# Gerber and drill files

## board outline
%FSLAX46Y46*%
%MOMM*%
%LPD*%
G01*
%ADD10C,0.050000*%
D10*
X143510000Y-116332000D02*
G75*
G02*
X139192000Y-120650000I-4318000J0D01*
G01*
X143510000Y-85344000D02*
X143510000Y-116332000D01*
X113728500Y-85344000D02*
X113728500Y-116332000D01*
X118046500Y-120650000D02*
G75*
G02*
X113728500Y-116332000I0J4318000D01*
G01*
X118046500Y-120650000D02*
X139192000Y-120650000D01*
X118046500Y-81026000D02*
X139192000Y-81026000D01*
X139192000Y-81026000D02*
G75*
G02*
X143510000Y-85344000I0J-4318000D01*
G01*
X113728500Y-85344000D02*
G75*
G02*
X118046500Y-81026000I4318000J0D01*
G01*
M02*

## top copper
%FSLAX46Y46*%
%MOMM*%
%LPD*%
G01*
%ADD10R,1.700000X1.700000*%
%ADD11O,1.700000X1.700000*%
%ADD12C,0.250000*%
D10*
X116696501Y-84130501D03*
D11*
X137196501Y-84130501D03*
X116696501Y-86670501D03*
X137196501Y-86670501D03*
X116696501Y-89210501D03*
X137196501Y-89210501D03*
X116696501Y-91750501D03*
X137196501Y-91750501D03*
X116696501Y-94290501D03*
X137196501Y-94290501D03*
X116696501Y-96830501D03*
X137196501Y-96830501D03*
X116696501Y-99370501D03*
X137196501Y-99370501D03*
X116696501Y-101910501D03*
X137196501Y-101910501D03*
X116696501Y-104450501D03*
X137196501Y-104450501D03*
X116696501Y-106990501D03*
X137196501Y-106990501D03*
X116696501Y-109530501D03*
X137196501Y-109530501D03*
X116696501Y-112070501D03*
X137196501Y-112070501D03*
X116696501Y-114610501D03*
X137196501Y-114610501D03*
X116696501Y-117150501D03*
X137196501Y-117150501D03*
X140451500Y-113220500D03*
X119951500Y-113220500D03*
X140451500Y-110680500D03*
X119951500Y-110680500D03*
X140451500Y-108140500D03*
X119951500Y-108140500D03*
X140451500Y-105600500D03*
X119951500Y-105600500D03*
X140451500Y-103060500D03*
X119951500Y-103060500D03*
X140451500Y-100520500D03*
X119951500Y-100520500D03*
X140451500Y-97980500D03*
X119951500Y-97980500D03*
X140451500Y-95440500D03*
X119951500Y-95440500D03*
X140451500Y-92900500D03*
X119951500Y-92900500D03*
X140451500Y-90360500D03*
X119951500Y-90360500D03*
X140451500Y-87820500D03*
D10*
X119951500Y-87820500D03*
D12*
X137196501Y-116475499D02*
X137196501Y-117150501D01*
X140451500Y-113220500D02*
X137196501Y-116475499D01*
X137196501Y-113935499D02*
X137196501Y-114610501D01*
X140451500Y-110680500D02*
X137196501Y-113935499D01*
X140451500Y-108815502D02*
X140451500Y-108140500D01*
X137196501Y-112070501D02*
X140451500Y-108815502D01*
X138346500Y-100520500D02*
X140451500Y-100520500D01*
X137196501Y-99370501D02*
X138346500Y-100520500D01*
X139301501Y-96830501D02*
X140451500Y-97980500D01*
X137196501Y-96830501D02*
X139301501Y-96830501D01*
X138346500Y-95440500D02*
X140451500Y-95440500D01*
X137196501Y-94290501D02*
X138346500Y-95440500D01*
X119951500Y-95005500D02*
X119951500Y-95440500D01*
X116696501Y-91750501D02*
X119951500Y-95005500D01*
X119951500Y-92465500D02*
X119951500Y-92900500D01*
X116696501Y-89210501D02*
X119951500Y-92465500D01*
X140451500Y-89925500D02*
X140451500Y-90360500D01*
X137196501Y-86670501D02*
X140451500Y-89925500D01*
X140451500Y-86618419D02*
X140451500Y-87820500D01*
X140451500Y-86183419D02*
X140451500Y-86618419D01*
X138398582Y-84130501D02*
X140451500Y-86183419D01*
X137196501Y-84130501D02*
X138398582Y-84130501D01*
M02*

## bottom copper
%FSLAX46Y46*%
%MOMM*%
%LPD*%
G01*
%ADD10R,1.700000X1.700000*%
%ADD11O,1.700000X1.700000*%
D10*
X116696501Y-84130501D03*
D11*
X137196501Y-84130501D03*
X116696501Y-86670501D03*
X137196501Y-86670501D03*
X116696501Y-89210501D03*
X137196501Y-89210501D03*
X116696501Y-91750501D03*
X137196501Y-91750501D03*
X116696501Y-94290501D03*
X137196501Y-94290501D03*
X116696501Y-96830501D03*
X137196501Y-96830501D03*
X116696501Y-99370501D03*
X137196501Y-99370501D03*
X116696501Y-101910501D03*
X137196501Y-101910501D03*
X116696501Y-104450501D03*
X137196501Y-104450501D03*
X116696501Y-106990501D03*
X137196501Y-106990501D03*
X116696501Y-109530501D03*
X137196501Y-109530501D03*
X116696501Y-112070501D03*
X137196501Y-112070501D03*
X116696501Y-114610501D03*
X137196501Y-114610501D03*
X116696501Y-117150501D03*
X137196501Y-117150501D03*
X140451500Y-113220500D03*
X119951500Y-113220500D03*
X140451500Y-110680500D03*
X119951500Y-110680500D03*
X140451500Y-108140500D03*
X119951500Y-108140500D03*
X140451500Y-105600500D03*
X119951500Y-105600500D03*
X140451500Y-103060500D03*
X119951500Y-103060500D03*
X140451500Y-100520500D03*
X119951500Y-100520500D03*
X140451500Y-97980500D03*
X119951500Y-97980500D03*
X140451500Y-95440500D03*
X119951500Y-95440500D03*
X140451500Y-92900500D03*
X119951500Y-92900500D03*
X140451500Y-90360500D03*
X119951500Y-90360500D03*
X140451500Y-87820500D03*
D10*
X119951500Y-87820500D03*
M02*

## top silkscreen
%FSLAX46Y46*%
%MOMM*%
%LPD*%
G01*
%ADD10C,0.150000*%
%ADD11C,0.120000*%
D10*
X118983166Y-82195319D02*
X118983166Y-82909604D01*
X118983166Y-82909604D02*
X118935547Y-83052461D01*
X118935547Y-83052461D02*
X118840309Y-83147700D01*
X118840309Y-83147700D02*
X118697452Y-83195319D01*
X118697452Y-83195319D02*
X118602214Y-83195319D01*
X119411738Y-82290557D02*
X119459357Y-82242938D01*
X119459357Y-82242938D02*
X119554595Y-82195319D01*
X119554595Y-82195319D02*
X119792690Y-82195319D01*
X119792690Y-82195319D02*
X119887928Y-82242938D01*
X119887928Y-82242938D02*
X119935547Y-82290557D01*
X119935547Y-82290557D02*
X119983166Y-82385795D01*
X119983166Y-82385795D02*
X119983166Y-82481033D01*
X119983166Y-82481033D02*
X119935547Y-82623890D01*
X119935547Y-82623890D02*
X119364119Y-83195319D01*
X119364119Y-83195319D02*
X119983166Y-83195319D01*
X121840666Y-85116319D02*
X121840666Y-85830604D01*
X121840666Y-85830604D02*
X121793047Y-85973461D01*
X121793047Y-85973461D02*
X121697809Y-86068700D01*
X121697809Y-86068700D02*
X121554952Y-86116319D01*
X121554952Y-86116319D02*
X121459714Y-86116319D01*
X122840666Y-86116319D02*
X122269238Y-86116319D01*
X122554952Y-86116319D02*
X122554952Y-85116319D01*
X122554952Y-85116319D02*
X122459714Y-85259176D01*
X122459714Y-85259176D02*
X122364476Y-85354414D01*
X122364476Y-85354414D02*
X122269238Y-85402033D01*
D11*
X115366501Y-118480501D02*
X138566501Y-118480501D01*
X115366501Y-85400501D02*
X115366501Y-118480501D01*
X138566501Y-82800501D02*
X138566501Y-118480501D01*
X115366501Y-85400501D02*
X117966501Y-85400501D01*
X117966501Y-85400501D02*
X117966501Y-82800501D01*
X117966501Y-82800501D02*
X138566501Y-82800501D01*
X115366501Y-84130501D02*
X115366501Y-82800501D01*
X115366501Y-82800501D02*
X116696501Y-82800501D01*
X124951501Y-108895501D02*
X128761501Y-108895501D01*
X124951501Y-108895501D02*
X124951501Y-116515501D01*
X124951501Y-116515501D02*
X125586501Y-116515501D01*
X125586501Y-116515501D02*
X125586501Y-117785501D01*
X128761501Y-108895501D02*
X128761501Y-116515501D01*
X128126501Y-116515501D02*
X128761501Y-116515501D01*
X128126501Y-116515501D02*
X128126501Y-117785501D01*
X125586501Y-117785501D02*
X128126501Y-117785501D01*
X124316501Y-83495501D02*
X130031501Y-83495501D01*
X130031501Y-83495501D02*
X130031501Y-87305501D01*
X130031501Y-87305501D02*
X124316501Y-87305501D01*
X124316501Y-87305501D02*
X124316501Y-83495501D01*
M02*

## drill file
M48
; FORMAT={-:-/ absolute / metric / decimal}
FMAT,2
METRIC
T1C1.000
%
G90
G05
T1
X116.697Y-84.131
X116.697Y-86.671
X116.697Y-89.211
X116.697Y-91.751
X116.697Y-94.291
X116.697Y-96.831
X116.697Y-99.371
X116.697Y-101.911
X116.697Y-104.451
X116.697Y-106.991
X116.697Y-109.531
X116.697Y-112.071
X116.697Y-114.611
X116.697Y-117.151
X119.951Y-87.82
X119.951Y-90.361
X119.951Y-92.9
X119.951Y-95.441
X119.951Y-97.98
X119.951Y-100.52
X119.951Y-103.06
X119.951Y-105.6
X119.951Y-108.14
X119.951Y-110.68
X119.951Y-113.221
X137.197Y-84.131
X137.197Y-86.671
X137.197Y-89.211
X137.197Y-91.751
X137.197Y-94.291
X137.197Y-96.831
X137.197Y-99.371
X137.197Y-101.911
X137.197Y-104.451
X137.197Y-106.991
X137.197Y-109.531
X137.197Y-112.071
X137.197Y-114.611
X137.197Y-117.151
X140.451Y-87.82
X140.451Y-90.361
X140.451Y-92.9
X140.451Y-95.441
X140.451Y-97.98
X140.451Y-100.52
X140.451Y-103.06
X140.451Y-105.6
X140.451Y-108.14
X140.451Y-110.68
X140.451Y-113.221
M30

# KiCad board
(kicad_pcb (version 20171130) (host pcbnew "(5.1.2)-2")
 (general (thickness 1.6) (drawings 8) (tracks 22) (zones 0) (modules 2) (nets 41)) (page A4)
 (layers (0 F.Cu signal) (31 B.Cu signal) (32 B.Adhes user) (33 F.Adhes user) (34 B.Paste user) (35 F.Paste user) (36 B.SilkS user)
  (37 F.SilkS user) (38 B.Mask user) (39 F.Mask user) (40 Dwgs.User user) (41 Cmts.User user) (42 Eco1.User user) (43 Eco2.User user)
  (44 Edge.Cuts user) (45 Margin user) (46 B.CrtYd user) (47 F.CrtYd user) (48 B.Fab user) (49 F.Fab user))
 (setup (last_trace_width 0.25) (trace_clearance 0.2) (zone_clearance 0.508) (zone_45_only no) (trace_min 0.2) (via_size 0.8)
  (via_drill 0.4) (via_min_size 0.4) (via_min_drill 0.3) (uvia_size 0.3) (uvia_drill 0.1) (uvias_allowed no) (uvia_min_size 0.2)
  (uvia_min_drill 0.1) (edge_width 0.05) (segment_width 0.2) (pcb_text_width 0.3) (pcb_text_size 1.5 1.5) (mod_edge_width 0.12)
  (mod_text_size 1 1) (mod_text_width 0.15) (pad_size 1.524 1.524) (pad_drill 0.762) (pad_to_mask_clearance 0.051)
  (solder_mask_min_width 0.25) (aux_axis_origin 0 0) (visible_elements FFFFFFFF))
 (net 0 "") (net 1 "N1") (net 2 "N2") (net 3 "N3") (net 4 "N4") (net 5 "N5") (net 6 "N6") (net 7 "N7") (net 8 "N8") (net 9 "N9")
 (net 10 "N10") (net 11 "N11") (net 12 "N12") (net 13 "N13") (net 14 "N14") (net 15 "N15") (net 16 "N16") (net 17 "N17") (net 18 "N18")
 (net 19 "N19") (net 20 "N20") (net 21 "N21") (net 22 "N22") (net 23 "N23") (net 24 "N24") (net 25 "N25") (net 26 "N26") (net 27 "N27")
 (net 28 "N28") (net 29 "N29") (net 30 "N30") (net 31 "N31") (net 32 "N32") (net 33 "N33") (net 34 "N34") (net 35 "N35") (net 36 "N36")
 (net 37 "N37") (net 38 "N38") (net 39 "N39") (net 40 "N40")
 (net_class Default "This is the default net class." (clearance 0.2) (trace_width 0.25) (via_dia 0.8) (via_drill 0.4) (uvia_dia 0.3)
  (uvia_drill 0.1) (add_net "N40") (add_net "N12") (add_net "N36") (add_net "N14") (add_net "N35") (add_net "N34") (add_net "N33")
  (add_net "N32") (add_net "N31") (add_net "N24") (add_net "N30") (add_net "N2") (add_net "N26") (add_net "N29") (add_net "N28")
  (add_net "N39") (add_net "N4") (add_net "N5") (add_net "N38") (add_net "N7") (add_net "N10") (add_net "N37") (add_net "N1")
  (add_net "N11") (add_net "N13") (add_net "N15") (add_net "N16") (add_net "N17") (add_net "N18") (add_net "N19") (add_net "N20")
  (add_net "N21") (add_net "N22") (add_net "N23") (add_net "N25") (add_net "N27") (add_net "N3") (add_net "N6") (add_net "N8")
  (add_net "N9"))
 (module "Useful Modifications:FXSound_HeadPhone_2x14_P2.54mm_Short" (layer F.Cu) (at 116.696501 84.130501)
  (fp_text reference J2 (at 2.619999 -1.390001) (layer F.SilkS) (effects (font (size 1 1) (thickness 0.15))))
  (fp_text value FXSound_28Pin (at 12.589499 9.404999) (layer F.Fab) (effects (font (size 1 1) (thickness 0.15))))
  (fp_line (start -1.33 34.35) (end 21.87 34.35) (layer F.SilkS) (width 0.12))
  (fp_line (start -1.33 1.27) (end -1.33 34.35) (layer F.SilkS) (width 0.12))
  (fp_line (start 21.87 -1.33) (end 21.87 34.35) (layer F.SilkS) (width 0.12))
  (fp_line (start -1.33 1.27) (end 1.27 1.27) (layer F.SilkS) (width 0.12))
  (fp_line (start 1.27 1.27) (end 1.27 -1.33) (layer F.SilkS) (width 0.12))
  (fp_line (start 1.27 -1.33) (end 21.87 -1.33) (layer F.SilkS) (width 0.12))
  (fp_line (start -1.33 0) (end -1.33 -1.33) (layer F.SilkS) (width 0.12))
  (fp_line (start -1.33 -1.33) (end 0 -1.33) (layer F.SilkS) (width 0.12))
  (fp_line (start 8.255 24.765) (end 12.065 24.765) (layer F.SilkS) (width 0.12))
  (fp_line (start 8.255 24.765) (end 8.255 32.385) (layer F.SilkS) (width 0.12))
  (fp_line (start 8.255 32.385) (end 8.89 32.385) (layer F.SilkS) (width 0.12))
  (fp_line (start 8.89 32.385) (end 8.89 33.655) (layer F.SilkS) (width 0.12))
  (fp_line (start 12.065 24.765) (end 12.065 32.385) (layer F.SilkS) (width 0.12))
  (fp_line (start 11.43 32.385) (end 12.065 32.385) (layer F.SilkS) (width 0.12))
  (fp_line (start 11.43 32.385) (end 11.43 33.655) (layer F.SilkS) (width 0.12))
  (fp_line (start 8.89 33.655) (end 11.43 33.655) (layer F.SilkS) (width 0.12))
  (fp_line (start 7.62 -0.635) (end 13.335 -0.635) (layer F.SilkS) (width 0.12))
  (fp_line (start 13.335 -0.635) (end 13.335 3.175) (layer F.SilkS) (width 0.12))
  (fp_line (start 13.335 3.175) (end 7.62 3.175) (layer F.SilkS) (width 0.12))
  (fp_line (start 7.62 3.175) (end 7.62 -0.635) (layer F.SilkS) (width 0.12))
  (pad 1 thru_hole rect (at 0 0) (size 1.7 1.7) (drill 1) (layers *.Cu *.Mask) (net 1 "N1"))
  (pad 2 thru_hole oval (at 20.5 0) (size 1.7 1.7) (drill 1) (layers *.Cu *.Mask) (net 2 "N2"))
  (pad 3 thru_hole oval (at 0 2.54) (size 1.7 1.7) (drill 1) (layers *.Cu *.Mask) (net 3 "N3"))
  (pad 4 thru_hole oval (at 20.5 2.54) (size 1.7 1.7) (drill 1) (layers *.Cu *.Mask) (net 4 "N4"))
  (pad 5 thru_hole oval (at 0 5.08) (size 1.7 1.7) (drill 1) (layers *.Cu *.Mask) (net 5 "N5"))
  (pad 6 thru_hole oval (at 20.5 5.08) (size 1.7 1.7) (drill 1) (layers *.Cu *.Mask) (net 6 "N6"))
  (pad 7 thru_hole oval (at 0 7.62) (size 1.7 1.7) (drill 1) (layers *.Cu *.Mask) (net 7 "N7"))
  (pad 8 thru_hole oval (at 20.5 7.62) (size 1.7 1.7) (drill 1) (layers *.Cu *.Mask) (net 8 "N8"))
  (pad 9 thru_hole oval (at 0 10.16) (size 1.7 1.7) (drill 1) (layers *.Cu *.Mask) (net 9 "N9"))
  (pad 10 thru_hole oval (at 20.5 10.16) (size 1.7 1.7) (drill 1) (layers *.Cu *.Mask) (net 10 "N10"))
  (pad 11 thru_hole oval (at 0 12.7) (size 1.7 1.7) (drill 1) (layers *.Cu *.Mask) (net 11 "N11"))
  (pad 12 thru_hole oval (at 20.5 12.7) (size 1.7 1.7) (drill 1) (layers *.Cu *.Mask) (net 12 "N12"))
  (pad 13 thru_hole oval (at 0 15.24) (size 1.7 1.7) (drill 1) (layers *.Cu *.Mask) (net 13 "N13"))
  (pad 14 thru_hole oval (at 20.5 15.24) (size 1.7 1.7) (drill 1) (layers *.Cu *.Mask) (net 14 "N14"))
  (pad 15 thru_hole oval (at 0 17.78) (size 1.7 1.7) (drill 1) (layers *.Cu *.Mask) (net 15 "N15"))
  (pad 16 thru_hole oval (at 20.5 17.78) (size 1.7 1.7) (drill 1) (layers *.Cu *.Mask) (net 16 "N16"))
  (pad 17 thru_hole oval (at 0 20.32) (size 1.7 1.7) (drill 1) (layers *.Cu *.Mask) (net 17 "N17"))
  (pad 18 thru_hole oval (at 20.5 20.32) (size 1.7 1.7) (drill 1) (layers *.Cu *.Mask) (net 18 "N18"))
  (pad 19 thru_hole oval (at 0 22.86) (size 1.7 1.7) (drill 1) (layers *.Cu *.Mask) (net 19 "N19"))
  (pad 20 thru_hole oval (at 20.5 22.86) (size 1.7 1.7) (drill 1) (layers *.Cu *.Mask) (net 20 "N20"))
  (pad 21 thru_hole oval (at 0 25.4) (size 1.7 1.7) (drill 1) (layers *.Cu *.Mask) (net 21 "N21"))
  (pad 22 thru_hole oval (at 20.5 25.4) (size 1.7 1.7) (drill 1) (layers *.Cu *.Mask) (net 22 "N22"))
  (pad 23 thru_hole oval (at 0 27.94) (size 1.7 1.7) (drill 1) (layers *.Cu *.Mask) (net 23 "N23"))
  (pad 24 thru_hole oval (at 20.5 27.94) (size 1.7 1.7) (drill 1) (layers *.Cu *.Mask) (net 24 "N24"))
  (pad 25 thru_hole oval (at 0 30.48) (size 1.7 1.7) (drill 1) (layers *.Cu *.Mask) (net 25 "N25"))
  (pad 26 thru_hole oval (at 20.5 30.48) (size 1.7 1.7) (drill 1) (layers *.Cu *.Mask) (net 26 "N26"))
  (pad 27 thru_hole oval (at 0 33.02) (size 1.7 1.7) (drill 1) (layers *.Cu *.Mask) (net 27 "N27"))
  (pad 28 thru_hole oval (at 20.5 33.02) (size 1.7 1.7) (drill 1) (layers *.Cu *.Mask) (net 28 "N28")))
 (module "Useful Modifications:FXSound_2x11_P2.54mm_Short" (layer F.Cu) (at 119.9515 87.8205)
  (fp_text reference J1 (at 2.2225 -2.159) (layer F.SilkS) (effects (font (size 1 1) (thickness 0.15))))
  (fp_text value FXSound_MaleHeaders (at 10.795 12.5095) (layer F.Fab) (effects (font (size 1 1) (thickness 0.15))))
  (pad 22 thru_hole oval (at 20.5 25.4) (size 1.7 1.7) (drill 1) (layers *.Cu *.Mask) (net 28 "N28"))
  (pad 21 thru_hole oval (at 0 25.4) (size 1.7 1.7) (drill 1) (layers *.Cu *.Mask) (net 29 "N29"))
  (pad 20 thru_hole oval (at 20.5 22.86) (size 1.7 1.7) (drill 1) (layers *.Cu *.Mask) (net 26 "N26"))
  (pad 19 thru_hole oval (at 0 22.86) (size 1.7 1.7) (drill 1) (layers *.Cu *.Mask) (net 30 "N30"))
  (pad 18 thru_hole oval (at 20.5 20.32) (size 1.7 1.7) (drill 1) (layers *.Cu *.Mask) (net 24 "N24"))
  (pad 17 thru_hole oval (at 0 20.32) (size 1.7 1.7) (drill 1) (layers *.Cu *.Mask) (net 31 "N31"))
  (pad 16 thru_hole oval (at 20.5 17.78) (size 1.7 1.7) (drill 1) (layers *.Cu *.Mask) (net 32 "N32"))
  (pad 15 thru_hole oval (at 0 17.78) (size 1.7 1.7) (drill 1) (layers *.Cu *.Mask) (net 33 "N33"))
  (pad 14 thru_hole oval (at 20.5 15.24) (size 1.7 1.7) (drill 1) (layers *.Cu *.Mask) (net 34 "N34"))
  (pad 13 thru_hole oval (at 0 15.24) (size 1.7 1.7) (drill 1) (layers *.Cu *.Mask) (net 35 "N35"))
  (pad 12 thru_hole oval (at 20.5 12.7) (size 1.7 1.7) (drill 1) (layers *.Cu *.Mask) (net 14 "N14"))
  (pad 11 thru_hole oval (at 0 12.7) (size 1.7 1.7) (drill 1) (layers *.Cu *.Mask) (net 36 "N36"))
  (pad 10 thru_hole oval (at 20.5 10.16) (size 1.7 1.7) (drill 1) (layers *.Cu *.Mask) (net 12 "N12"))
  (pad 9 thru_hole oval (at 0 10.16) (size 1.7 1.7) (drill 1) (layers *.Cu *.Mask) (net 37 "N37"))
  (pad 8 thru_hole oval (at 20.5 7.62) (size 1.7 1.7) (drill 1) (layers *.Cu *.Mask) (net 10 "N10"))
  (pad 7 thru_hole oval (at 0 7.62) (size 1.7 1.7) (drill 1) (layers *.Cu *.Mask) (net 7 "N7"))
  (pad 6 thru_hole oval (at 20.5 5.08) (size 1.7 1.7) (drill 1) (layers *.Cu *.Mask) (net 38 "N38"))
  (pad 5 thru_hole oval (at 0 5.08) (size 1.7 1.7) (drill 1) (layers *.Cu *.Mask) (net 5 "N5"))
  (pad 4 thru_hole oval (at 20.5 2.54) (size 1.7 1.7) (drill 1) (layers *.Cu *.Mask) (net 4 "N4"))
  (pad 3 thru_hole oval (at 0 2.54) (size 1.7 1.7) (drill 1) (layers *.Cu *.Mask) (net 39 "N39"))
  (pad 2 thru_hole oval (at 20.5 0) (size 1.7 1.7) (drill 1) (layers *.Cu *.Mask) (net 2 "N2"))
  (pad 1 thru_hole rect (at 0 0) (size 1.7 1.7) (drill 1) (layers *.Cu *.Mask) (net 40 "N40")))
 (gr_arc (start 139.192 116.332) (end 139.192 120.65) (angle -90) (layer Edge.Cuts) (width 0.05))
 (gr_line (start 143.51 85.344) (end 143.51 116.332) (layer Edge.Cuts) (width 0.05))
 (gr_line (start 113.7285 85.344) (end 113.7285 116.332) (layer Edge.Cuts) (width 0.05))
 (gr_arc (start 118.0465 116.332) (end 113.7285 116.332) (angle -90) (layer Edge.Cuts) (width 0.05))
 (gr_line (start 118.0465 120.65) (end 139.192 120.65) (layer Edge.Cuts) (width 0.05))
 (gr_line (start 118.0465 81.026) (end 139.192 81.026) (layer Edge.Cuts) (width 0.05))
 (gr_arc (start 139.192 85.344) (end 143.51 85.344) (angle -90) (layer Edge.Cuts) (width 0.05))
 (gr_arc (start 118.0465 85.344) (end 118.0465 81.026) (angle -90) (layer Edge.Cuts) (width 0.05))
 (segment (start 137.196501 116.475499) (end 137.196501 117.150501) (width 0.25) (layer F.Cu) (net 28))
 (segment (start 140.4515 113.2205) (end 137.196501 116.475499) (width 0.25) (layer F.Cu) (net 28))
 (segment (start 137.196501 113.935499) (end 137.196501 114.610501) (width 0.25) (layer F.Cu) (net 26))
 (segment (start 140.4515 110.6805) (end 137.196501 113.935499) (width 0.25) (layer F.Cu) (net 26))
 (segment (start 140.4515 108.815502) (end 140.4515 108.1405) (width 0.25) (layer F.Cu) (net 24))
 (segment (start 137.196501 112.070501) (end 140.4515 108.815502) (width 0.25) (layer F.Cu) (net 24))
 (segment (start 138.3465 100.5205) (end 140.4515 100.5205) (width 0.25) (layer F.Cu) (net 14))
 (segment (start 137.196501 99.370501) (end 138.3465 100.5205) (width 0.25) (layer F.Cu) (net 14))
 (segment (start 139.301501 96.830501) (end 140.4515 97.9805) (width 0.25) (layer F.Cu) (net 12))
 (segment (start 137.196501 96.830501) (end 139.301501 96.830501) (width 0.25) (layer F.Cu) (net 12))
 (segment (start 138.3465 95.4405) (end 140.4515 95.4405) (width 0.25) (layer F.Cu) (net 10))
 (segment (start 137.196501 94.290501) (end 138.3465 95.4405) (width 0.25) (layer F.Cu) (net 10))
 (segment (start 119.9515 95.0055) (end 119.9515 95.4405) (width 0.25) (layer F.Cu) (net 7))
 (segment (start 116.696501 91.750501) (end 119.9515 95.0055) (width 0.25) (layer F.Cu) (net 7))
 (segment (start 119.9515 92.4655) (end 119.9515 92.9005) (width 0.25) (layer F.Cu) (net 5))
 (segment (start 116.696501 89.210501) (end 119.9515 92.4655) (width 0.25) (layer F.Cu) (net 5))
 (segment (start 140.4515 89.9255) (end 140.4515 90.3605) (width 0.25) (layer F.Cu) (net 4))
 (segment (start 137.196501 86.670501) (end 140.4515 89.9255) (width 0.25) (layer F.Cu) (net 4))
 (segment (start 140.4515 86.618419) (end 140.4515 87.8205) (width 0.25) (layer F.Cu) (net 2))
 (segment (start 140.4515 86.183419) (end 140.4515 86.618419) (width 0.25) (layer F.Cu) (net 2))
 (segment (start 138.398582 84.130501) (end 140.4515 86.183419) (width 0.25) (layer F.Cu) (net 2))
 (segment (start 137.196501 84.130501) (end 138.398582 84.130501) (width 0.25) (layer F.Cu) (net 2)))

